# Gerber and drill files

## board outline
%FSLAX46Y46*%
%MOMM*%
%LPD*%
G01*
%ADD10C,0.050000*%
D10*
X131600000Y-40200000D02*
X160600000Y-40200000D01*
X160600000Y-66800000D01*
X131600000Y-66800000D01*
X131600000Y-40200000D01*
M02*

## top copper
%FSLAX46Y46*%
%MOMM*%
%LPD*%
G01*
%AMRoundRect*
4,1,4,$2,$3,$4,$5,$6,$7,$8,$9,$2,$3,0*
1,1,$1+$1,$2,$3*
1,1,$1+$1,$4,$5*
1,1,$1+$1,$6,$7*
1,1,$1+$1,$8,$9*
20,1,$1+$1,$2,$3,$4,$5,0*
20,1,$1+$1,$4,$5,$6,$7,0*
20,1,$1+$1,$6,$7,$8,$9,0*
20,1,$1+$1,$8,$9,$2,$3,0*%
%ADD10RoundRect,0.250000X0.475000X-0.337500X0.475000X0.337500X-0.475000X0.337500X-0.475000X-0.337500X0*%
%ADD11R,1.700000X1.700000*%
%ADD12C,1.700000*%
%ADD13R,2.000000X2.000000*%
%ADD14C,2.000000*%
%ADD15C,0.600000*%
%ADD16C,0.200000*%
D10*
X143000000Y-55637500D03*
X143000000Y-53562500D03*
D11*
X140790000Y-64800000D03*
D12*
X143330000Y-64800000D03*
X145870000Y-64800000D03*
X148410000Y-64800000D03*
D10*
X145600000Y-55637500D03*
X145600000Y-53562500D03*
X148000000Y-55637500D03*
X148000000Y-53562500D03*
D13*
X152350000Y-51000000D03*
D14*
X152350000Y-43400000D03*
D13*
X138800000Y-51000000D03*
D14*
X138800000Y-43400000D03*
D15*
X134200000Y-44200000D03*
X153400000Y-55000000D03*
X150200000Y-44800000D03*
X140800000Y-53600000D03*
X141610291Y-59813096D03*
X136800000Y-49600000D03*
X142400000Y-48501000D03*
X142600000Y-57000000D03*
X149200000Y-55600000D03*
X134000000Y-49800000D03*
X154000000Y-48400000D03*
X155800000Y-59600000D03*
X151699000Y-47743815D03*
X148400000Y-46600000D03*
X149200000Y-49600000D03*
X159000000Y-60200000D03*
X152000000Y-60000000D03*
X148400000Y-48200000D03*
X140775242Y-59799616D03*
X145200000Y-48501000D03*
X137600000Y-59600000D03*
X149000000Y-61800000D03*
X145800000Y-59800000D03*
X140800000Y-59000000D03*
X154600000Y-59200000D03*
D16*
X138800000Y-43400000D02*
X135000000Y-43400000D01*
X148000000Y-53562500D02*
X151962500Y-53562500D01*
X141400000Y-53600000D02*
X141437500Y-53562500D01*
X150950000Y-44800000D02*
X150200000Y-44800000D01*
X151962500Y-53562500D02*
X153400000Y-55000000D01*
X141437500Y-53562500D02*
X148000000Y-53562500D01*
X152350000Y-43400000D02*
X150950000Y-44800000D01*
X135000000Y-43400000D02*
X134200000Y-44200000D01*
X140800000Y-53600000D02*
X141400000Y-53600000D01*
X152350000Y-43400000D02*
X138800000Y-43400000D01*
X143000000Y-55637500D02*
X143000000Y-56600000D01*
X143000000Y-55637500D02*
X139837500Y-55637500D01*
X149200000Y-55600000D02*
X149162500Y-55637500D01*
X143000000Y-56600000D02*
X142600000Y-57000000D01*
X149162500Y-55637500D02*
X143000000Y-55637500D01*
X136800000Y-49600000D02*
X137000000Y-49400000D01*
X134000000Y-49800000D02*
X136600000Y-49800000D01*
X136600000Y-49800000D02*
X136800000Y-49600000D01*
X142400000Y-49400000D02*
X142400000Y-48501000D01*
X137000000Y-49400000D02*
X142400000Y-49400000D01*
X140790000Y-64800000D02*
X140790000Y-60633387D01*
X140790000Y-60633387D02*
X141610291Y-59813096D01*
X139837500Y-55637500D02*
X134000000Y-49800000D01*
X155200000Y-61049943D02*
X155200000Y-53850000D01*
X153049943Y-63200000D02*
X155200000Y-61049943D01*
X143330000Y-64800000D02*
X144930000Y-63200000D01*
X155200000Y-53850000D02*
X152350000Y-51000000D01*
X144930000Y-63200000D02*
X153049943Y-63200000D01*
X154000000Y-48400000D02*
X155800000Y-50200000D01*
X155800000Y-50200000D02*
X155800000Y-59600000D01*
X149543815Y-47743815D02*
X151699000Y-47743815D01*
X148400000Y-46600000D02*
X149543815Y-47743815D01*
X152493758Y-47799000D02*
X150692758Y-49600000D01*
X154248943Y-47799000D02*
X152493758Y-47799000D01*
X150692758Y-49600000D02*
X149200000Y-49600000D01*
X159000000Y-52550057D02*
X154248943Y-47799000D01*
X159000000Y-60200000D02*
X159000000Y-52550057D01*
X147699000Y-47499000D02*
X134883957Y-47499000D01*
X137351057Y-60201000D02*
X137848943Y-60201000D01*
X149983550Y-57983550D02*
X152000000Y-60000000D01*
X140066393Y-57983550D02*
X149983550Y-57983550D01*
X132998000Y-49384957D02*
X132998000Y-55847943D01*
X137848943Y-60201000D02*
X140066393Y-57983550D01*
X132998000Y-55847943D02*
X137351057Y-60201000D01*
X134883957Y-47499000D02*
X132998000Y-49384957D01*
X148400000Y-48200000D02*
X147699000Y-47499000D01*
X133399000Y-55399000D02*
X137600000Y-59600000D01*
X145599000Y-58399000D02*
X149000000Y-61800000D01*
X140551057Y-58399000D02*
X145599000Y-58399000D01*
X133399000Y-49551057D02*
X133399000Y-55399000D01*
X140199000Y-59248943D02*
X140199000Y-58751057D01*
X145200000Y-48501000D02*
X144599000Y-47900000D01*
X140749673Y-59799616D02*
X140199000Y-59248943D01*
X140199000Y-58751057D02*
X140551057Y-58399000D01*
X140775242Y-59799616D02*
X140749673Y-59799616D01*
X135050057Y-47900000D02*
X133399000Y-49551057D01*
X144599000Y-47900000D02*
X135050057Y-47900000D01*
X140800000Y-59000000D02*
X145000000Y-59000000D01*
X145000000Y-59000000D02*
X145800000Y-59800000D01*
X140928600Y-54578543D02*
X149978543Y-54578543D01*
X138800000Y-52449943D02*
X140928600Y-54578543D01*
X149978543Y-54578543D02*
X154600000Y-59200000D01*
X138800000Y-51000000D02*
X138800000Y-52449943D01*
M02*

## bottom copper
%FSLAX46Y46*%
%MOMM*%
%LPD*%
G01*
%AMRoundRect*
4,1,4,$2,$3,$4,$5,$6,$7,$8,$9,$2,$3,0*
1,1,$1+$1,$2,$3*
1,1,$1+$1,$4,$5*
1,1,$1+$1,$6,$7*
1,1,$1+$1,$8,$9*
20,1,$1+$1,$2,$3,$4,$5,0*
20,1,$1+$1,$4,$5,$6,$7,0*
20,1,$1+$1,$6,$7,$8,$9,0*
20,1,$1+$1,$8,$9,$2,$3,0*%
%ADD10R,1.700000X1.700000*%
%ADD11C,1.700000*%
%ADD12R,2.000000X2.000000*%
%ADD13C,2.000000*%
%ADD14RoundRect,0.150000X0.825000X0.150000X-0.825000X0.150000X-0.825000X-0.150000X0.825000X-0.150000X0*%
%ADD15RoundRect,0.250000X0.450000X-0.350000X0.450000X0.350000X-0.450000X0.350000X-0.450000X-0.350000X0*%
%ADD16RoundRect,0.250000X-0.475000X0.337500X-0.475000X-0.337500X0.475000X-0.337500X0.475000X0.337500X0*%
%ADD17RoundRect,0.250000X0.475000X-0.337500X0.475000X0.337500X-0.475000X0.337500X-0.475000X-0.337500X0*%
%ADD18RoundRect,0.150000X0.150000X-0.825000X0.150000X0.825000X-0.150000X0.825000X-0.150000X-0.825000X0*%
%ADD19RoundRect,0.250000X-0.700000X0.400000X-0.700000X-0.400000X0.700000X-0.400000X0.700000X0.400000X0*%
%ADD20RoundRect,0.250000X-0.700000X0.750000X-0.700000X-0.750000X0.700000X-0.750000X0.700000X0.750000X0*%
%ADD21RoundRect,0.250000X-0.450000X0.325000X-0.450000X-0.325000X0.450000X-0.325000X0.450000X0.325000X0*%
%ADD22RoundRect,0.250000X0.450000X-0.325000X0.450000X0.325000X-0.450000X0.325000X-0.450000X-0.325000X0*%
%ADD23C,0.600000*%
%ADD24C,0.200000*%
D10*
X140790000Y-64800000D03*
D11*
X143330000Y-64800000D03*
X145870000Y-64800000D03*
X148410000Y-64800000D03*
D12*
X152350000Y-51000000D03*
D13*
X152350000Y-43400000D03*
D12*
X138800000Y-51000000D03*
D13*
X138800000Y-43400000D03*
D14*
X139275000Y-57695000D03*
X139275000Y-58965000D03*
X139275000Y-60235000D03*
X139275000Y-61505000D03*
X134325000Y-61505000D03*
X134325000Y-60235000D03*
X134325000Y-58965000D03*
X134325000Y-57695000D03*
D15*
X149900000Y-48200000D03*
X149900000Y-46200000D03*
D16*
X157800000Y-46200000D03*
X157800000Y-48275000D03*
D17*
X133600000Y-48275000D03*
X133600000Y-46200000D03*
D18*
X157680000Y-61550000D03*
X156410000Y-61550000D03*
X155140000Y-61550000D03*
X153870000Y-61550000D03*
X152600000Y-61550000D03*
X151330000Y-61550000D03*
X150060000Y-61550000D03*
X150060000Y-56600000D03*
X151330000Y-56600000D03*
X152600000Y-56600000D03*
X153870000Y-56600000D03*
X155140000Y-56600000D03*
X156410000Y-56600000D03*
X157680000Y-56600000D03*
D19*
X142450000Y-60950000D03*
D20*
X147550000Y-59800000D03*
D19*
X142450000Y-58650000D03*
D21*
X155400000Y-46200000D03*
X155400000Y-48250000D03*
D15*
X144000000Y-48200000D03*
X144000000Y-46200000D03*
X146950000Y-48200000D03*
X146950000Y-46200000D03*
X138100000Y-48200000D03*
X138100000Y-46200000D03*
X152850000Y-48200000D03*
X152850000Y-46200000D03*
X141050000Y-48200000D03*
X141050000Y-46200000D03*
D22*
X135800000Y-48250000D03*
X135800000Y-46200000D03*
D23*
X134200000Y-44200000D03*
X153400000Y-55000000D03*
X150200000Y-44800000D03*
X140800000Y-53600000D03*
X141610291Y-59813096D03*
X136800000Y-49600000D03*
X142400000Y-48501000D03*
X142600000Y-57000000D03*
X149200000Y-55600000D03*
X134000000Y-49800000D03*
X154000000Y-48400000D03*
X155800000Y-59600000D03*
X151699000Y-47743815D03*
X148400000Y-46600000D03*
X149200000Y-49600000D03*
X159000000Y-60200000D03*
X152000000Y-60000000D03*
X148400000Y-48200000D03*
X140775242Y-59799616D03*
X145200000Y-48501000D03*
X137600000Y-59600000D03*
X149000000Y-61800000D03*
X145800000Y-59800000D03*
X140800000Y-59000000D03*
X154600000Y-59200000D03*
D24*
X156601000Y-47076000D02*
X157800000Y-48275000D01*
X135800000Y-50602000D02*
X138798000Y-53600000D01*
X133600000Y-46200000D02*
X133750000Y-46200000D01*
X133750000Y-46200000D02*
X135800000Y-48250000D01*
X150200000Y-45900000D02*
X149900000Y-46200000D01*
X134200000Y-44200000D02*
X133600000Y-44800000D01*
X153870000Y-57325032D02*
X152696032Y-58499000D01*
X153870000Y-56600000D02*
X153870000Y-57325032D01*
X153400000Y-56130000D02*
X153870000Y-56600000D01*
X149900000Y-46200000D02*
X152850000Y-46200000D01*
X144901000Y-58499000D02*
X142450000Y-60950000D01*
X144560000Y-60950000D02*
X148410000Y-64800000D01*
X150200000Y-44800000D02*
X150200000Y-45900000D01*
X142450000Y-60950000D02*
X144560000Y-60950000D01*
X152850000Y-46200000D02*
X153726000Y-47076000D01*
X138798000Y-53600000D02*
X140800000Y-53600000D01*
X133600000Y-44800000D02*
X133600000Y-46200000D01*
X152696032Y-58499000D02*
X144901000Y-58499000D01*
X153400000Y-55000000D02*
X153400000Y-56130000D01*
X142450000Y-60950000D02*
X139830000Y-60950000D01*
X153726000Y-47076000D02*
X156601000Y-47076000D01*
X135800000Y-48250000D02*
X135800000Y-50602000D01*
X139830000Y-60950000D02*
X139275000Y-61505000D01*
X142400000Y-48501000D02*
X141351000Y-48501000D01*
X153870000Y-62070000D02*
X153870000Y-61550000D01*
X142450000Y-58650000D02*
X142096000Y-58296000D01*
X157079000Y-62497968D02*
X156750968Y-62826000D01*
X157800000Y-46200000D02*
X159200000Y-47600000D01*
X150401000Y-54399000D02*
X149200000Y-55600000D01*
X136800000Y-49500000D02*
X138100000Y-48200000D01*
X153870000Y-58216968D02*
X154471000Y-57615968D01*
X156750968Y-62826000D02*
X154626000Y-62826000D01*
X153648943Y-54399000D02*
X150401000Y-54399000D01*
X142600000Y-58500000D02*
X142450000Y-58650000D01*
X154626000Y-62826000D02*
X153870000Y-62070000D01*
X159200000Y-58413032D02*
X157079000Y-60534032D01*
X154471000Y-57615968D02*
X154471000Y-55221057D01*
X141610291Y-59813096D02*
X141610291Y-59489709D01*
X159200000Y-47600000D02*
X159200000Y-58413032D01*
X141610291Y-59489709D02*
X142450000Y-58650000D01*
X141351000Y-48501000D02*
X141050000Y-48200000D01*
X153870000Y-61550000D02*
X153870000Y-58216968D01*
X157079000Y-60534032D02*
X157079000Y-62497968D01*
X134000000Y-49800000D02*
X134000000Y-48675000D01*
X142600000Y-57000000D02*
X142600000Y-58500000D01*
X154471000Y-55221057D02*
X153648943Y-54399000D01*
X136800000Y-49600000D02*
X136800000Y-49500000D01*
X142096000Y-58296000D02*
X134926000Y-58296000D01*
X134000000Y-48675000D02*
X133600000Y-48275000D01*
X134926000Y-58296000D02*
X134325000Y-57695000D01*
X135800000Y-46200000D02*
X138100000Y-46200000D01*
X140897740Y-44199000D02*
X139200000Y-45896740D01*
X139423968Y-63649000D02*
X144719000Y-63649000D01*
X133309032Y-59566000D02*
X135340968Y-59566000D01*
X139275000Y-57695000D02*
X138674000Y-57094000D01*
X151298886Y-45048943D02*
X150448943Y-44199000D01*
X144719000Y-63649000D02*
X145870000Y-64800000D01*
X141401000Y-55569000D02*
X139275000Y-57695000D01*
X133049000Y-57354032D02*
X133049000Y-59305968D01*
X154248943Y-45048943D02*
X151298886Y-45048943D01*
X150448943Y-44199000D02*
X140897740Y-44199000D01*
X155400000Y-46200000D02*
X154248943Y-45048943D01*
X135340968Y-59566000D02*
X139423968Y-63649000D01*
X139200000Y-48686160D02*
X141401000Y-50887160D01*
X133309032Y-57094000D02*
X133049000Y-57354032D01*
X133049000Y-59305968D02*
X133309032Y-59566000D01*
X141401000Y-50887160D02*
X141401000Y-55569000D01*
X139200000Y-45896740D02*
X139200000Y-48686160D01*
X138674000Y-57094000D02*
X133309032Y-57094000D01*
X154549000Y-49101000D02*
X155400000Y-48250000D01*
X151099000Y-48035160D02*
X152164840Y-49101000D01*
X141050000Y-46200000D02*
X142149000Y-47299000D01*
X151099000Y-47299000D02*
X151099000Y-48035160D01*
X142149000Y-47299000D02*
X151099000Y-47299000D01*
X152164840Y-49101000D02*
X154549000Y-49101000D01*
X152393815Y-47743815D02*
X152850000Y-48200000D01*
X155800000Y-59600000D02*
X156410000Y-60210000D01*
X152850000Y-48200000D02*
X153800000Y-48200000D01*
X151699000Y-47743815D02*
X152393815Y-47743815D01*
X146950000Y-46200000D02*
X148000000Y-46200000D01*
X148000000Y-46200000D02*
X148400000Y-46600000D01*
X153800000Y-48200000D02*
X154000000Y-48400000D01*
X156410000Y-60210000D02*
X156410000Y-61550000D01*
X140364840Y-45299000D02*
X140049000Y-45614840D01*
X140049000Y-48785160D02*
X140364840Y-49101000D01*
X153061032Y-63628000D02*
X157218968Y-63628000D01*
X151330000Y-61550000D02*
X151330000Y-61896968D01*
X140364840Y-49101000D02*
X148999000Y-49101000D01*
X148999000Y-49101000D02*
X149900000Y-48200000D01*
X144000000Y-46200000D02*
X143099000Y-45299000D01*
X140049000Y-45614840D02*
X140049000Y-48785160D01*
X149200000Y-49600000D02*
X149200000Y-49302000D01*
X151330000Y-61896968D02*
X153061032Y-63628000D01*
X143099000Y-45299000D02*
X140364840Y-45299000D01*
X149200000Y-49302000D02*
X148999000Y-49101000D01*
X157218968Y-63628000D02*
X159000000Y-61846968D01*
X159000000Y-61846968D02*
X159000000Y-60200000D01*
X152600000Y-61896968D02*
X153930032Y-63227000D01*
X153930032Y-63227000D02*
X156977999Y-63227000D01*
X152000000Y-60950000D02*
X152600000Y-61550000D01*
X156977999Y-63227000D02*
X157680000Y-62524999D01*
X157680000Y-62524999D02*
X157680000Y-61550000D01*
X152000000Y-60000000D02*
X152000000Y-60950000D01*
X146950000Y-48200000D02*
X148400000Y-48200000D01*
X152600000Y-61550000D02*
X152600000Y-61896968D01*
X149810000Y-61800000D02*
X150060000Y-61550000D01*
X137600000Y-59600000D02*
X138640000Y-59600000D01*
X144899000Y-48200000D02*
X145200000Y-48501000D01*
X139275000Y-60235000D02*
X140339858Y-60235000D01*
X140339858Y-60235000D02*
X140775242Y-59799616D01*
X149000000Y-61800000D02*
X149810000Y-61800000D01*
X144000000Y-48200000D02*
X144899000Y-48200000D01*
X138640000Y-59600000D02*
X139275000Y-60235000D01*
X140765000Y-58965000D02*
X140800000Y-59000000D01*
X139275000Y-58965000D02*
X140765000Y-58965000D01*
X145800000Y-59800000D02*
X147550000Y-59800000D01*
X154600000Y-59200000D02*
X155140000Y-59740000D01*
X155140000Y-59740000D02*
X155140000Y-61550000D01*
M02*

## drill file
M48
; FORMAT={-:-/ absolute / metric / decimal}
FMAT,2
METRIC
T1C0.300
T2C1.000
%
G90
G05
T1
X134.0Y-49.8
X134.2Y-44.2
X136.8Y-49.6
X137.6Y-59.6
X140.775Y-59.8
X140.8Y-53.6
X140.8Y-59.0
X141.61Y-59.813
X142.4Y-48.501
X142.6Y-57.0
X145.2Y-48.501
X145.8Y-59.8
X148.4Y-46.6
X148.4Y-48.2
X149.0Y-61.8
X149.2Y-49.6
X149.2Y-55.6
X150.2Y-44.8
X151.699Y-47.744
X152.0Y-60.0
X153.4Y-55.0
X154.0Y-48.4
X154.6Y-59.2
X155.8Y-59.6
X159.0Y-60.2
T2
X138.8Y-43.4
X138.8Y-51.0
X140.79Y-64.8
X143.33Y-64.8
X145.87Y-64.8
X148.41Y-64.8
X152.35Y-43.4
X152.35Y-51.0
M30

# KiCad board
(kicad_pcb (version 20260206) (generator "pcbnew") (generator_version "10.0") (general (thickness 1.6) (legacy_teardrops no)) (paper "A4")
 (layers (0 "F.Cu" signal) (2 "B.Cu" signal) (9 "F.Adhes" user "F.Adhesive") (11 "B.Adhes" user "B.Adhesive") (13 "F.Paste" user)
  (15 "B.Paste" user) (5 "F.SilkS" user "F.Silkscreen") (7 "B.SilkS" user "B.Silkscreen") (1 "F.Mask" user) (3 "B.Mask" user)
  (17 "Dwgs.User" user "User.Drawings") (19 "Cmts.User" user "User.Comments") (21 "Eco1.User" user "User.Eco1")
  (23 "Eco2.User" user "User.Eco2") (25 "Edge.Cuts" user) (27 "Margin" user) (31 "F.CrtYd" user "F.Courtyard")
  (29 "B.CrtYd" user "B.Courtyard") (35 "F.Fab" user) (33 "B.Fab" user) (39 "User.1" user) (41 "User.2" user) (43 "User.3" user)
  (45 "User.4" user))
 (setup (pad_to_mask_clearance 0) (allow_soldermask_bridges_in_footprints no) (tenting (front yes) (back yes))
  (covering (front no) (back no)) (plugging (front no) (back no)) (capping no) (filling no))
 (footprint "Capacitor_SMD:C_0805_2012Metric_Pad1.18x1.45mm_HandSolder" (layer "F.Cu") (at 143 54.6 90)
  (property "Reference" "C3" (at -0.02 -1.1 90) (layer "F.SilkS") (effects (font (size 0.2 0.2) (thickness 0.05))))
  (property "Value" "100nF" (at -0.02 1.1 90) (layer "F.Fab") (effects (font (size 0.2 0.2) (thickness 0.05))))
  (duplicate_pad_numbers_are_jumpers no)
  (pad "1" smd roundrect (at -1.0375 0 90) (size 1.175 1.45) (layers "F.Cu" "F.Mask" "F.Paste") (roundrect_rratio 0.212766) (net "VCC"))
  (pad "2" smd roundrect (at 1.0375 0 90) (size 1.175 1.45) (layers "F.Cu" "F.Mask" "F.Paste") (roundrect_rratio 0.212766) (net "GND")))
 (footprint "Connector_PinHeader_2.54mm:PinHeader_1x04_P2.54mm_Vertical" (layer "F.Cu") (at 140.79 64.8 90)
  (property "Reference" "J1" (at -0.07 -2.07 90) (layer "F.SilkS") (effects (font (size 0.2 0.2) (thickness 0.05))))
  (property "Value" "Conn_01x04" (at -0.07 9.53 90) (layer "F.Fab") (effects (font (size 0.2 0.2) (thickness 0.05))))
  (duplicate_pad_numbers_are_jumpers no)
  (pad "1" thru_hole rect (at 0 0 90) (size 1.7 1.7) (drill 1) (layers "*.Cu" "*.Mask") (remove_unused_layers no) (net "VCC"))
  (pad "2" thru_hole circle (at 0 2.54 90) (size 1.7 1.7) (drill 1) (layers "*.Cu" "*.Mask") (remove_unused_layers no)
   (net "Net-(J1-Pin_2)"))
  (pad "3" thru_hole circle (at 0 5.08 90) (size 1.7 1.7) (drill 1) (layers "*.Cu" "*.Mask") (remove_unused_layers no) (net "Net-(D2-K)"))
  (pad "4" thru_hole circle (at 0 7.62 90) (size 1.7 1.7) (drill 1) (layers "*.Cu" "*.Mask") (remove_unused_layers no) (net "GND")))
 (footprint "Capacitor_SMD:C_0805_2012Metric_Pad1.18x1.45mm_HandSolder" (layer "F.Cu") (at 145.6 54.6 90)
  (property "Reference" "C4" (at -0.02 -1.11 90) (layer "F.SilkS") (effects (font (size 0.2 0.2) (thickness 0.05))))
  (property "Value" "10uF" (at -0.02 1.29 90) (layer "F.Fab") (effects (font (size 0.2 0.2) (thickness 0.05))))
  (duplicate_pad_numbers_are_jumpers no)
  (pad "1" smd roundrect (at -1.0375 0 90) (size 1.175 1.45) (layers "F.Cu" "F.Mask" "F.Paste") (roundrect_rratio 0.212766) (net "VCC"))
  (pad "2" smd roundrect (at 1.0375 0 90) (size 1.175 1.45) (layers "F.Cu" "F.Mask" "F.Paste") (roundrect_rratio 0.212766) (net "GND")))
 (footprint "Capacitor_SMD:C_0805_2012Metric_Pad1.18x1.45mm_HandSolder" (layer "F.Cu") (at 148 54.6 90)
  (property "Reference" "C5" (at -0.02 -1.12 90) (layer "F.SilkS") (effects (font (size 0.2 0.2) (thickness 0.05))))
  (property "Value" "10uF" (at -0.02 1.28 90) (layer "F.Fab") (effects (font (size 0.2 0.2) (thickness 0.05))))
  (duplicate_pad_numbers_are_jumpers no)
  (pad "1" smd roundrect (at -1.0375 0 90) (size 1.175 1.45) (layers "F.Cu" "F.Mask" "F.Paste") (roundrect_rratio 0.212766) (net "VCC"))
  (pad "2" smd roundrect (at 1.0375 0 90) (size 1.175 1.45) (layers "F.Cu" "F.Mask" "F.Paste") (roundrect_rratio 0.212766) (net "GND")))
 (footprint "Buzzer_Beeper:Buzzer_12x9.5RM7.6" (layer "F.Cu") (at 152.35 51 90)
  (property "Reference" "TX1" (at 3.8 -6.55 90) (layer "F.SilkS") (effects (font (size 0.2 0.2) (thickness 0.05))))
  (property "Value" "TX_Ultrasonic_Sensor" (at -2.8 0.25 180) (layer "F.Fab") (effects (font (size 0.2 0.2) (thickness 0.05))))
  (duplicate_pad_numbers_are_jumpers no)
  (pad "1" thru_hole rect (at 0 0 90) (size 2 2) (drill 1) (layers "*.Cu" "*.Mask") (remove_unused_layers no) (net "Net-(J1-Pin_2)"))
  (pad "2" thru_hole circle (at 7.6 0 90) (size 2 2) (drill 1) (layers "*.Cu" "*.Mask") (remove_unused_layers no) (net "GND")))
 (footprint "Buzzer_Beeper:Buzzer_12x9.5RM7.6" (layer "F.Cu") (at 138.8 51 90)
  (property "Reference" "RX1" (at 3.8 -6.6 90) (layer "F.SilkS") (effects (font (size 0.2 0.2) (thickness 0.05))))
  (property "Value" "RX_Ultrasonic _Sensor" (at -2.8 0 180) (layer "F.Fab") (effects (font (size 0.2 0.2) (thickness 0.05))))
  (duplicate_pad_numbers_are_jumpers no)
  (pad "1" thru_hole rect (at 0 0 90) (size 2 2) (drill 1) (layers "*.Cu" "*.Mask") (remove_unused_layers no) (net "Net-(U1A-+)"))
  (pad "2" thru_hole circle (at 7.6 0 90) (size 2 2) (drill 1) (layers "*.Cu" "*.Mask") (remove_unused_layers no) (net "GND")))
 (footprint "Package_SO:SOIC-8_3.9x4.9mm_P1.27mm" (layer "B.Cu") (at 136.8 59.6 180)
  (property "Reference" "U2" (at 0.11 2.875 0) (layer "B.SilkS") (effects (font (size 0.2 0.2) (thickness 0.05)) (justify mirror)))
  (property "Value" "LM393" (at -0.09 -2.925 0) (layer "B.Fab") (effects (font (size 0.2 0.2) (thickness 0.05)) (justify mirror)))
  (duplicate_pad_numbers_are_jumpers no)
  (pad "1" smd roundrect (at -2.475 1.905 180) (size 1.95 0.6) (layers "B.Cu" "B.Mask" "B.Paste") (roundrect_rratio 0.25) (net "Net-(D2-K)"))
  (pad "2" smd roundrect (at -2.475 0.635 180) (size 1.95 0.6) (layers "B.Cu" "B.Mask" "B.Paste") (roundrect_rratio 0.25)
   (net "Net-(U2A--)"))
  (pad "3" smd roundrect (at -2.475 -0.635 180) (size 1.95 0.6) (layers "B.Cu" "B.Mask" "B.Paste") (roundrect_rratio 0.25)
   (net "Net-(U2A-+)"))
  (pad "4" smd roundrect (at -2.475 -1.905 180) (size 1.95 0.6) (layers "B.Cu" "B.Mask" "B.Paste") (roundrect_rratio 0.25) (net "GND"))
  (pad "5" smd roundrect (at 2.475 -1.905 180) (size 1.95 0.6) (layers "B.Cu" "B.Mask" "B.Paste") (roundrect_rratio 0.25))
  (pad "6" smd roundrect (at 2.475 -0.635 180) (size 1.95 0.6) (layers "B.Cu" "B.Mask" "B.Paste") (roundrect_rratio 0.25))
  (pad "7" smd roundrect (at 2.475 0.635 180) (size 1.95 0.6) (layers "B.Cu" "B.Mask" "B.Paste") (roundrect_rratio 0.25))
  (pad "8" smd roundrect (at 2.475 1.905 180) (size 1.95 0.6) (layers "B.Cu" "B.Mask" "B.Paste") (roundrect_rratio 0.25) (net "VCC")))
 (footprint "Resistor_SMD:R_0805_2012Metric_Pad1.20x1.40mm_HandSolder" (layer "B.Cu") (at 149.9 47.2 90)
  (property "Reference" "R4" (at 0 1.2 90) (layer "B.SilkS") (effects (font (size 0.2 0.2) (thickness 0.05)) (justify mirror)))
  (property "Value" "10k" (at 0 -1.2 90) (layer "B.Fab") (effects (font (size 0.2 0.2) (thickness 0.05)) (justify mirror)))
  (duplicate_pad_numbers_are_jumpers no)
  (pad "1" smd roundrect (at -1 0 90) (size 1.2 1.4) (layers "B.Cu" "B.Mask" "B.Paste") (roundrect_rratio 0.208333) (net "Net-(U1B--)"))
  (pad "2" smd roundrect (at 1 0 90) (size 1.2 1.4) (layers "B.Cu" "B.Mask" "B.Paste") (roundrect_rratio 0.208333) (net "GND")))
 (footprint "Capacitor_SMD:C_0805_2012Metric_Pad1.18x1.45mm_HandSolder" (layer "B.Cu") (at 157.8 47.2375 -90)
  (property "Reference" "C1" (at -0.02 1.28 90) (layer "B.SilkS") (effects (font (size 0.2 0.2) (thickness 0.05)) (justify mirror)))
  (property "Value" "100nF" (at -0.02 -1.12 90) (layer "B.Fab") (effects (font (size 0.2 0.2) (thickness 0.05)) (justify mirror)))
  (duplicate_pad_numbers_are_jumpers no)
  (pad "1" smd roundrect (at -1.0375 0 270) (size 1.175 1.45) (layers "B.Cu" "B.Mask" "B.Paste") (roundrect_rratio 0.212766) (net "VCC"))
  (pad "2" smd roundrect (at 1.0375 0 270) (size 1.175 1.45) (layers "B.Cu" "B.Mask" "B.Paste") (roundrect_rratio 0.212766) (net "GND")))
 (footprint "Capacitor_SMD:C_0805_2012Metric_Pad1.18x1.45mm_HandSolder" (layer "B.Cu") (at 133.6 47.2375 90)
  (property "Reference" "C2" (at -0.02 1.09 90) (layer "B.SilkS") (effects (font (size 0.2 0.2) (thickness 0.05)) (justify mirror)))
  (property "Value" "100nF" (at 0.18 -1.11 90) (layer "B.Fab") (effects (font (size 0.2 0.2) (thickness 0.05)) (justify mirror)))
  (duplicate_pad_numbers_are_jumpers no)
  (pad "1" smd roundrect (at -1.0375 0 90) (size 1.175 1.45) (layers "B.Cu" "B.Mask" "B.Paste") (roundrect_rratio 0.212766) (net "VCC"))
  (pad "2" smd roundrect (at 1.0375 0 90) (size 1.175 1.45) (layers "B.Cu" "B.Mask" "B.Paste") (roundrect_rratio 0.212766) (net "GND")))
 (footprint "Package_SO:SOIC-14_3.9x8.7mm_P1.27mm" (layer "B.Cu") (at 153.87 59.075 90)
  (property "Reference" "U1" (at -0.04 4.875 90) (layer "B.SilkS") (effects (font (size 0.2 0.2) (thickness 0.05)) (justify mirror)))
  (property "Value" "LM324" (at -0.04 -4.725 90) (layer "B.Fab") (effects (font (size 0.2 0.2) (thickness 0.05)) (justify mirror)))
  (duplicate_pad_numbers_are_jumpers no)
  (pad "1" smd roundrect (at -2.475 3.81 90) (size 1.95 0.6) (layers "B.Cu" "B.Mask" "B.Paste") (roundrect_rratio 0.25) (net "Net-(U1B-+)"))
  (pad "2" smd roundrect (at -2.475 2.54 90) (size 1.95 0.6) (layers "B.Cu" "B.Mask" "B.Paste") (roundrect_rratio 0.25) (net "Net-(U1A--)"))
  (pad "3" smd roundrect (at -2.475 1.27 90) (size 1.95 0.6) (layers "B.Cu" "B.Mask" "B.Paste") (roundrect_rratio 0.25) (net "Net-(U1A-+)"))
  (pad "4" smd roundrect (at -2.475 0 90) (size 1.95 0.6) (layers "B.Cu" "B.Mask" "B.Paste") (roundrect_rratio 0.25) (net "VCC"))
  (pad "5" smd roundrect (at -2.475 -1.27 90) (size 1.95 0.6) (layers "B.Cu" "B.Mask" "B.Paste") (roundrect_rratio 0.25) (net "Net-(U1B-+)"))
  (pad "6" smd roundrect (at -2.475 -2.54 90) (size 1.95 0.6) (layers "B.Cu" "B.Mask" "B.Paste") (roundrect_rratio 0.25) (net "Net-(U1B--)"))
  (pad "7" smd roundrect (at -2.475 -3.81 90) (size 1.95 0.6) (layers "B.Cu" "B.Mask" "B.Paste") (roundrect_rratio 0.25) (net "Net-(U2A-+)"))
  (pad "8" smd roundrect (at 2.475 -3.81 90) (size 1.95 0.6) (layers "B.Cu" "B.Mask" "B.Paste") (roundrect_rratio 0.25))
  (pad "9" smd roundrect (at 2.475 -2.54 90) (size 1.95 0.6) (layers "B.Cu" "B.Mask" "B.Paste") (roundrect_rratio 0.25))
  (pad "10" smd roundrect (at 2.475 -1.27 90) (size 1.95 0.6) (layers "B.Cu" "B.Mask" "B.Paste") (roundrect_rratio 0.25))
  (pad "11" smd roundrect (at 2.475 0 90) (size 1.95 0.6) (layers "B.Cu" "B.Mask" "B.Paste") (roundrect_rratio 0.25) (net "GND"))
  (pad "12" smd roundrect (at 2.475 1.27 90) (size 1.95 0.6) (layers "B.Cu" "B.Mask" "B.Paste") (roundrect_rratio 0.25))
  (pad "13" smd roundrect (at 2.475 2.54 90) (size 1.95 0.6) (layers "B.Cu" "B.Mask" "B.Paste") (roundrect_rratio 0.25))
  (pad "14" smd roundrect (at 2.475 3.81 90) (size 1.95 0.6) (layers "B.Cu" "B.Mask" "B.Paste") (roundrect_rratio 0.25)))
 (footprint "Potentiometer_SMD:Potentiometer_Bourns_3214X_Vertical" (layer "B.Cu") (at 145 59.8 -90)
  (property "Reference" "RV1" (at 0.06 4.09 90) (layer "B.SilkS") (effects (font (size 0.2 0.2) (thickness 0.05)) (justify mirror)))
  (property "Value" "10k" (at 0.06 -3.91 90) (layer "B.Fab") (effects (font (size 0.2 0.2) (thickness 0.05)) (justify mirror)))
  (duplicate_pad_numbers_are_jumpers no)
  (pad "1" smd roundrect (at 1.15 2.55 270) (size 1.3 1.9) (layers "B.Cu" "B.Mask" "B.Paste") (roundrect_rratio 0.192308) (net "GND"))
  (pad "2" smd roundrect (at 0 -2.55 270) (size 2 1.9) (layers "B.Cu" "B.Mask" "B.Paste") (roundrect_rratio 0.131579) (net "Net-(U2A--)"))
  (pad "3" smd roundrect (at -1.15 2.55 270) (size 1.3 1.9) (layers "B.Cu" "B.Mask" "B.Paste") (roundrect_rratio 0.192308) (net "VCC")))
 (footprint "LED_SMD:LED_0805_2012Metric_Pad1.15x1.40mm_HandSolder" (layer "B.Cu") (at 155.4 47.225 -90)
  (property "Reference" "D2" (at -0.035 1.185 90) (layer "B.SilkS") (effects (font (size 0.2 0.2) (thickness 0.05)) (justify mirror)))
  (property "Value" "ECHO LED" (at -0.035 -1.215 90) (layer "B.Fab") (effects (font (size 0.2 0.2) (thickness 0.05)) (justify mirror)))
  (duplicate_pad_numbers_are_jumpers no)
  (pad "1" smd roundrect (at -1.025 0 270) (size 1.15 1.4) (layers "B.Cu" "B.Mask" "B.Paste") (roundrect_rratio 0.217391) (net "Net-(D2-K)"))
  (pad "2" smd roundrect (at 1.025 0 270) (size 1.15 1.4) (layers "B.Cu" "B.Mask" "B.Paste") (roundrect_rratio 0.217391) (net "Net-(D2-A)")))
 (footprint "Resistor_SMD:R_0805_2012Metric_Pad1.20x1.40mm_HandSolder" (layer "B.Cu") (at 144 47.2 90)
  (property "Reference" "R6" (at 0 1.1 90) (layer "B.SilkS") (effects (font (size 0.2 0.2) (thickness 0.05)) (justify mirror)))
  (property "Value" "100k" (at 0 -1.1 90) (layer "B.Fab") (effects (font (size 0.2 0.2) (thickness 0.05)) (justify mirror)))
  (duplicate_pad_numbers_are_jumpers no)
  (pad "1" smd roundrect (at -1 0 90) (size 1.2 1.4) (layers "B.Cu" "B.Mask" "B.Paste") (roundrect_rratio 0.208333) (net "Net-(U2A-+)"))
  (pad "2" smd roundrect (at 1 0 90) (size 1.2 1.4) (layers "B.Cu" "B.Mask" "B.Paste") (roundrect_rratio 0.208333) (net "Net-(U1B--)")))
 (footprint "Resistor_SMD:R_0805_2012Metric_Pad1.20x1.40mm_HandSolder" (layer "B.Cu") (at 146.95 47.2 90)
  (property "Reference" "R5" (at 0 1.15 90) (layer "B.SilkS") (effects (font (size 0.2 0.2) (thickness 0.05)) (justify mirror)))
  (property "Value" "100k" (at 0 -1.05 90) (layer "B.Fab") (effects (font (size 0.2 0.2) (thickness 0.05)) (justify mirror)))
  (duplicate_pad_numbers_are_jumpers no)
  (pad "1" smd roundrect (at -1 0 90) (size 1.2 1.4) (layers "B.Cu" "B.Mask" "B.Paste") (roundrect_rratio 0.208333) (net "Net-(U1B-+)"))
  (pad "2" smd roundrect (at 1 0 90) (size 1.2 1.4) (layers "B.Cu" "B.Mask" "B.Paste") (roundrect_rratio 0.208333) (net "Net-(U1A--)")))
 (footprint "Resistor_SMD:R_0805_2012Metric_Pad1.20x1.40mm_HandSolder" (layer "B.Cu") (at 138.1 47.2 90)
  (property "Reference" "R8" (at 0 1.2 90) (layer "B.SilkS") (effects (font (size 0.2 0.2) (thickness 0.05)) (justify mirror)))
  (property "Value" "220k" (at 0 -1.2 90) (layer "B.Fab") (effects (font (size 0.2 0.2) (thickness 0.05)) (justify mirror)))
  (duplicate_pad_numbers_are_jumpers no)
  (pad "1" smd roundrect (at -1 0 90) (size 1.2 1.4) (layers "B.Cu" "B.Mask" "B.Paste") (roundrect_rratio 0.208333) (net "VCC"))
  (pad "2" smd roundrect (at 1 0 90) (size 1.2 1.4) (layers "B.Cu" "B.Mask" "B.Paste") (roundrect_rratio 0.208333) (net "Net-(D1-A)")))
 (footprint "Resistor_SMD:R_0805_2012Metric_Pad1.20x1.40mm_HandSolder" (layer "B.Cu") (at 152.85 47.2 90)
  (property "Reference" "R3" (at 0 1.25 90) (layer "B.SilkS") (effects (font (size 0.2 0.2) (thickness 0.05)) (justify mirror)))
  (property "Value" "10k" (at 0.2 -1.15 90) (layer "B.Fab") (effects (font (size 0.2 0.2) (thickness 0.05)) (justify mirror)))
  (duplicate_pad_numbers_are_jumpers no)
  (pad "1" smd roundrect (at -1 0 90) (size 1.2 1.4) (layers "B.Cu" "B.Mask" "B.Paste") (roundrect_rratio 0.208333) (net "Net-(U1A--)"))
  (pad "2" smd roundrect (at 1 0 90) (size 1.2 1.4) (layers "B.Cu" "B.Mask" "B.Paste") (roundrect_rratio 0.208333) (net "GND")))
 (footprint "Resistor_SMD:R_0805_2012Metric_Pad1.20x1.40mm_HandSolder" (layer "B.Cu") (at 141.05 47.2 90)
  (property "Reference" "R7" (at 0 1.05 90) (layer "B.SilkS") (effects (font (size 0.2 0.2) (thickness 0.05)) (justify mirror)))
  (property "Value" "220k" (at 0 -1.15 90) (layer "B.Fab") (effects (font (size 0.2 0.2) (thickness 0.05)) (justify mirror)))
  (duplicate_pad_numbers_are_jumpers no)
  (pad "1" smd roundrect (at -1 0 90) (size 1.2 1.4) (layers "B.Cu" "B.Mask" "B.Paste") (roundrect_rratio 0.208333) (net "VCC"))
  (pad "2" smd roundrect (at 1 0 90) (size 1.2 1.4) (layers "B.Cu" "B.Mask" "B.Paste") (roundrect_rratio 0.208333) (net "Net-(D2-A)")))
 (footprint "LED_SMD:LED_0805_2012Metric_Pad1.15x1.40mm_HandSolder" (layer "B.Cu") (at 135.8 47.225 90)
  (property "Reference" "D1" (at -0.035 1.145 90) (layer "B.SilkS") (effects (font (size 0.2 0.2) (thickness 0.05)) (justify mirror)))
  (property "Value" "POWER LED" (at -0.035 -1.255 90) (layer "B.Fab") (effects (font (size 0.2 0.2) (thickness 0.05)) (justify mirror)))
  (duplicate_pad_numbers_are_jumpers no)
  (pad "1" smd roundrect (at -1.025 0 90) (size 1.15 1.4) (layers "B.Cu" "B.Mask" "B.Paste") (roundrect_rratio 0.217391) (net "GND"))
  (pad "2" smd roundrect (at 1.025 0 90) (size 1.15 1.4) (layers "B.Cu" "B.Mask" "B.Paste") (roundrect_rratio 0.217391) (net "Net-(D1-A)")))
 (gr_rect (start 131.6 40.2) (end 160.6 66.8) (stroke (width 0.05) (type default)) (fill no) (layer "Edge.Cuts"))
 (segment (start 138.8 43.4) (end 135 43.4) (width 0.2) (layer "F.Cu") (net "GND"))
 (segment (start 148 53.5625) (end 151.9625 53.5625) (width 0.2) (layer "F.Cu") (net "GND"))
 (segment (start 141.4 53.6) (end 141.4375 53.5625) (width 0.2) (layer "F.Cu") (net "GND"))
 (segment (start 150.95 44.8) (end 150.2 44.8) (width 0.2) (layer "F.Cu") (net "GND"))
 (segment (start 151.9625 53.5625) (end 153.4 55) (width 0.2) (layer "F.Cu") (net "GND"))
 (segment (start 141.4375 53.5625) (end 148 53.5625) (width 0.2) (layer "F.Cu") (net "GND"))
 (segment (start 152.35 43.4) (end 150.95 44.8) (width 0.2) (layer "F.Cu") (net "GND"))
 (segment (start 135 43.4) (end 134.2 44.2) (width 0.2) (layer "F.Cu") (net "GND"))
 (segment (start 140.8 53.6) (end 141.4 53.6) (width 0.2) (layer "F.Cu") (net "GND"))
 (segment (start 152.35 43.4) (end 138.8 43.4) (width 0.2) (layer "F.Cu") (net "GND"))
 (via (at 134.2 44.2) (size 0.6) (drill 0.3) (layers "F.Cu" "B.Cu") (capping no) (covering (front no) (back no))
  (plugging (front no) (back no)) (filling no) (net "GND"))
 (via (at 153.4 55) (size 0.6) (drill 0.3) (layers "F.Cu" "B.Cu") (capping no) (covering (front no) (back no))
  (plugging (front no) (back no)) (filling no) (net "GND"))
 (via (at 150.2 44.8) (size 0.6) (drill 0.3) (layers "F.Cu" "B.Cu") (capping no) (covering (front no) (back no))
  (plugging (front no) (back no)) (filling no) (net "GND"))
 (via (at 140.8 53.6) (size 0.6) (drill 0.3) (layers "F.Cu" "B.Cu") (capping no) (covering (front no) (back no))
  (plugging (front no) (back no)) (filling no) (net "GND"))
 (segment (start 156.601 47.076) (end 157.8 48.275) (width 0.2) (layer "B.Cu") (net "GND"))
 (segment (start 135.8 50.602) (end 138.798 53.6) (width 0.2) (layer "B.Cu") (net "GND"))
 (segment (start 133.6 46.2) (end 133.75 46.2) (width 0.2) (layer "B.Cu") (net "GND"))
 (segment (start 133.75 46.2) (end 135.8 48.25) (width 0.2) (layer "B.Cu") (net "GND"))
 (segment (start 150.2 45.9) (end 149.9 46.2) (width 0.2) (layer "B.Cu") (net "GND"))
 (segment (start 134.2 44.2) (end 133.6 44.8) (width 0.2) (layer "B.Cu") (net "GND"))
 (segment (start 153.87 57.325032) (end 152.696032 58.499) (width 0.2) (layer "B.Cu") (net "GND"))
 (segment (start 153.87 56.6) (end 153.87 57.325032) (width 0.2) (layer "B.Cu") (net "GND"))
 (segment (start 153.4 56.13) (end 153.87 56.6) (width 0.2) (layer "B.Cu") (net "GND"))
 (segment (start 149.9 46.2) (end 152.85 46.2) (width 0.2) (layer "B.Cu") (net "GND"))
 (segment (start 144.901 58.499) (end 142.45 60.95) (width 0.2) (layer "B.Cu") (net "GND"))
 (segment (start 144.56 60.95) (end 148.41 64.8) (width 0.2) (layer "B.Cu") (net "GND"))
 (segment (start 150.2 44.8) (end 150.2 45.9) (width 0.2) (layer "B.Cu") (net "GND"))
 (segment (start 142.45 60.95) (end 144.56 60.95) (width 0.2) (layer "B.Cu") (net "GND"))
 (segment (start 152.85 46.2) (end 153.726 47.076) (width 0.2) (layer "B.Cu") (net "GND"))
 (segment (start 138.798 53.6) (end 140.8 53.6) (width 0.2) (layer "B.Cu") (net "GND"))
 (segment (start 133.6 44.8) (end 133.6 46.2) (width 0.2) (layer "B.Cu") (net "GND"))
 (segment (start 152.696032 58.499) (end 144.901 58.499) (width 0.2) (layer "B.Cu") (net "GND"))
 (segment (start 153.4 55) (end 153.4 56.13) (width 0.2) (layer "B.Cu") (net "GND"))
 (segment (start 142.45 60.95) (end 139.83 60.95) (width 0.2) (layer "B.Cu") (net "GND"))
 (segment (start 153.726 47.076) (end 156.601 47.076) (width 0.2) (layer "B.Cu") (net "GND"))
 (segment (start 135.8 48.25) (end 135.8 50.602) (width 0.2) (layer "B.Cu") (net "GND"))
 (segment (start 139.83 60.95) (end 139.275 61.505) (width 0.2) (layer "B.Cu") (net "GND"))
 (segment (start 143 55.6375) (end 143 56.6) (width 0.2) (layer "F.Cu") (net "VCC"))
 (segment (start 143 55.6375) (end 139.8375 55.6375) (width 0.2) (layer "F.Cu") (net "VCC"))
 (segment (start 149.2 55.6) (end 149.1625 55.6375) (width 0.2) (layer "F.Cu") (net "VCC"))
 (segment (start 143 56.6) (end 142.6 57) (width 0.2) (layer "F.Cu") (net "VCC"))
 (segment (start 149.1625 55.6375) (end 143 55.6375) (width 0.2) (layer "F.Cu") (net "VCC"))
 (segment (start 136.8 49.6) (end 137 49.4) (width 0.2) (layer "F.Cu") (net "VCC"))
 (segment (start 134 49.8) (end 136.6 49.8) (width 0.2) (layer "F.Cu") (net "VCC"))
 (segment (start 136.6 49.8) (end 136.8 49.6) (width 0.2) (layer "F.Cu") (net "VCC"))
 (segment (start 142.4 49.4) (end 142.4 48.501) (width 0.2) (layer "F.Cu") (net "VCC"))
 (segment (start 137 49.4) (end 142.4 49.4) (width 0.2) (layer "F.Cu") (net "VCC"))
 (segment (start 140.79 64.8) (end 140.79 60.633387) (width 0.2) (layer "F.Cu") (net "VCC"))
 (segment (start 140.79 60.633387) (end 141.610291 59.813096) (width 0.2) (layer "F.Cu") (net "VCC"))
 (segment (start 139.8375 55.6375) (end 134 49.8) (width 0.2) (layer "F.Cu") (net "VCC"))
 (via (at 141.610291 59.813096) (size 0.6) (drill 0.3) (layers "F.Cu" "B.Cu") (capping no) (covering (front no) (back no))
  (plugging (front no) (back no)) (filling no) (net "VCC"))
 (via (at 136.8 49.6) (size 0.6) (drill 0.3) (layers "F.Cu" "B.Cu") (capping no) (covering (front no) (back no))
  (plugging (front no) (back no)) (filling no) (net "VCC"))
 (via (at 142.4 48.501) (size 0.6) (drill 0.3) (layers "F.Cu" "B.Cu") (capping no) (covering (front no) (back no))
  (plugging (front no) (back no)) (filling no) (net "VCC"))
 (via (at 142.6 57) (size 0.6) (drill 0.3) (layers "F.Cu" "B.Cu") (capping no) (covering (front no) (back no))
  (plugging (front no) (back no)) (filling no) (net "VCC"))
 (via (at 149.2 55.6) (size 0.6) (drill 0.3) (layers "F.Cu" "B.Cu") (capping no) (covering (front no) (back no))
  (plugging (front no) (back no)) (filling no) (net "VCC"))
 (via (at 134 49.8) (size 0.6) (drill 0.3) (layers "F.Cu" "B.Cu") (capping no) (covering (front no) (back no))
  (plugging (front no) (back no)) (filling no) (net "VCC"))
 (segment (start 142.4 48.501) (end 141.351 48.501) (width 0.2) (layer "B.Cu") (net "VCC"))
 (segment (start 153.87 62.07) (end 153.87 61.55) (width 0.2) (layer "B.Cu") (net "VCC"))
 (segment (start 142.45 58.65) (end 142.096 58.296) (width 0.2) (layer "B.Cu") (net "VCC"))
 (segment (start 157.079 62.497968) (end 156.750968 62.826) (width 0.2) (layer "B.Cu") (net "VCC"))
 (segment (start 157.8 46.2) (end 159.2 47.6) (width 0.2) (layer "B.Cu") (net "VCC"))
 (segment (start 150.401 54.399) (end 149.2 55.6) (width 0.2) (layer "B.Cu") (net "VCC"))
 (segment (start 136.8 49.5) (end 138.1 48.2) (width 0.2) (layer "B.Cu") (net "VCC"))
 (segment (start 153.87 58.216968) (end 154.471 57.615968) (width 0.2) (layer "B.Cu") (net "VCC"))
 (segment (start 156.750968 62.826) (end 154.626 62.826) (width 0.2) (layer "B.Cu") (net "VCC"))
 (segment (start 153.648943 54.399) (end 150.401 54.399) (width 0.2) (layer "B.Cu") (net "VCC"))
 (segment (start 142.6 58.5) (end 142.45 58.65) (width 0.2) (layer "B.Cu") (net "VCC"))
 (segment (start 154.626 62.826) (end 153.87 62.07) (width 0.2) (layer "B.Cu") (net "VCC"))
 (segment (start 159.2 58.413032) (end 157.079 60.534032) (width 0.2) (layer "B.Cu") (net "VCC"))
 (segment (start 154.471 57.615968) (end 154.471 55.221057) (width 0.2) (layer "B.Cu") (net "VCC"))
 (segment (start 141.610291 59.813096) (end 141.610291 59.489709) (width 0.2) (layer "B.Cu") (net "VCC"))
 (segment (start 159.2 47.6) (end 159.2 58.413032) (width 0.2) (layer "B.Cu") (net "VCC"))
 (segment (start 141.610291 59.489709) (end 142.45 58.65) (width 0.2) (layer "B.Cu") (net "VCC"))
 (segment (start 141.351 48.501) (end 141.05 48.2) (width 0.2) (layer "B.Cu") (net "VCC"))
 (segment (start 153.87 61.55) (end 153.87 58.216968) (width 0.2) (layer "B.Cu") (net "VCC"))
 (segment (start 157.079 60.534032) (end 157.079 62.497968) (width 0.2) (layer "B.Cu") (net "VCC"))
 (segment (start 134 49.8) (end 134 48.675) (width 0.2) (layer "B.Cu") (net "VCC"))
 (segment (start 142.6 57) (end 142.6 58.5) (width 0.2) (layer "B.Cu") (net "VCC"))
 (segment (start 154.471 55.221057) (end 153.648943 54.399) (width 0.2) (layer "B.Cu") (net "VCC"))
 (segment (start 136.8 49.6) (end 136.8 49.5) (width 0.2) (layer "B.Cu") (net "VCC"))
 (segment (start 142.096 58.296) (end 134.926 58.296) (width 0.2) (layer "B.Cu") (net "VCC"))
 (segment (start 134 48.675) (end 133.6 48.275) (width 0.2) (layer "B.Cu") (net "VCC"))
 (segment (start 134.926 58.296) (end 134.325 57.695) (width 0.2) (layer "B.Cu") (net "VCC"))
 (segment (start 135.8 46.2) (end 138.1 46.2) (width 0.2) (layer "B.Cu") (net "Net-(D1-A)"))
 (segment (start 140.89774 44.199) (end 139.2 45.89674) (width 0.2) (layer "B.Cu") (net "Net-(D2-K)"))
 (segment (start 139.423968 63.649) (end 144.719 63.649) (width 0.2) (layer "B.Cu") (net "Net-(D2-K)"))
 (segment (start 133.309032 59.566) (end 135.340968 59.566) (width 0.2) (layer "B.Cu") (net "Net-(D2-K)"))
 (segment (start 139.275 57.695) (end 138.674 57.094) (width 0.2) (layer "B.Cu") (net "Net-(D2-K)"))
 (segment (start 151.298886 45.048943) (end 150.448943 44.199) (width 0.2) (layer "B.Cu") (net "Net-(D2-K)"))
 (segment (start 144.719 63.649) (end 145.87 64.8) (width 0.2) (layer "B.Cu") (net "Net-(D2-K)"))
 (segment (start 141.401 55.569) (end 139.275 57.695) (width 0.2) (layer "B.Cu") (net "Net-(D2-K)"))
 (segment (start 133.049 57.354032) (end 133.049 59.305968) (width 0.2) (layer "B.Cu") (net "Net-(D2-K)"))
 (segment (start 154.248943 45.048943) (end 151.298886 45.048943) (width 0.2) (layer "B.Cu") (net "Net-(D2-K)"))
 (segment (start 150.448943 44.199) (end 140.89774 44.199) (width 0.2) (layer "B.Cu") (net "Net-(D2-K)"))
 (segment (start 155.4 46.2) (end 154.248943 45.048943) (width 0.2) (layer "B.Cu") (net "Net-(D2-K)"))
 (segment (start 135.340968 59.566) (end 139.423968 63.649) (width 0.2) (layer "B.Cu") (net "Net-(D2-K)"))
 (segment (start 139.2 48.68616) (end 141.401 50.88716) (width 0.2) (layer "B.Cu") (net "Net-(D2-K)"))
 (segment (start 133.309032 57.094) (end 133.049 57.354032) (width 0.2) (layer "B.Cu") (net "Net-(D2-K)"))
 (segment (start 133.049 59.305968) (end 133.309032 59.566) (width 0.2) (layer "B.Cu") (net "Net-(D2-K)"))
 (segment (start 141.401 50.88716) (end 141.401 55.569) (width 0.2) (layer "B.Cu") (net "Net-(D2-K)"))
 (segment (start 139.2 45.89674) (end 139.2 48.68616) (width 0.2) (layer "B.Cu") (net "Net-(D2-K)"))
 (segment (start 138.674 57.094) (end 133.309032 57.094) (width 0.2) (layer "B.Cu") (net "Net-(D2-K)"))
 (segment (start 154.549 49.101) (end 155.4 48.25) (width 0.2) (layer "B.Cu") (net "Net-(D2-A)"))
 (segment (start 151.099 48.03516) (end 152.16484 49.101) (width 0.2) (layer "B.Cu") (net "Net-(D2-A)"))
 (segment (start 141.05 46.2) (end 142.149 47.299) (width 0.2) (layer "B.Cu") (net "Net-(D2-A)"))
 (segment (start 151.099 47.299) (end 151.099 48.03516) (width 0.2) (layer "B.Cu") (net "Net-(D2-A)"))
 (segment (start 142.149 47.299) (end 151.099 47.299) (width 0.2) (layer "B.Cu") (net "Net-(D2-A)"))
 (segment (start 152.16484 49.101) (end 154.549 49.101) (width 0.2) (layer "B.Cu") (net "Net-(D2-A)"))
 (segment (start 155.2 61.049943) (end 155.2 53.85) (width 0.2) (layer "F.Cu") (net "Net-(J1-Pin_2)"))
 (segment (start 153.049943 63.2) (end 155.2 61.049943) (width 0.2) (layer "F.Cu") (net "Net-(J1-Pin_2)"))
 (segment (start 143.33 64.8) (end 144.93 63.2) (width 0.2) (layer "F.Cu") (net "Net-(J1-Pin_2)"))
 (segment (start 155.2 53.85) (end 152.35 51) (width 0.2) (layer "F.Cu") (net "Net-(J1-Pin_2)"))
 (segment (start 144.93 63.2) (end 153.049943 63.2) (width 0.2) (layer "F.Cu") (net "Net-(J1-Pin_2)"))
 (segment (start 154 48.4) (end 155.8 50.2) (width 0.2) (layer "F.Cu") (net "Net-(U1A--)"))
 (segment (start 155.8 50.2) (end 155.8 59.6) (width 0.2) (layer "F.Cu") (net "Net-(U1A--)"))
 (segment (start 149.543815 47.743815) (end 151.699 47.743815) (width 0.2) (layer "F.Cu") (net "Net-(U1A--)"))
 (segment (start 148.4 46.6) (end 149.543815 47.743815) (width 0.2) (layer "F.Cu") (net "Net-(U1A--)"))
 (via (at 154 48.4) (size 0.6) (drill 0.3) (layers "F.Cu" "B.Cu") (capping no) (covering (front no) (back no))
  (plugging (front no) (back no)) (filling no) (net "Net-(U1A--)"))
 (via (at 155.8 59.6) (size 0.6) (drill 0.3) (layers "F.Cu" "B.Cu") (capping no) (covering (front no) (back no))
  (plugging (front no) (back no)) (filling no) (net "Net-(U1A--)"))
 (via (at 151.699 47.743815) (size 0.6) (drill 0.3) (layers "F.Cu" "B.Cu") (capping no) (covering (front no) (back no))
  (plugging (front no) (back no)) (filling no) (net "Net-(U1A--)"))
 (via (at 148.4 46.6) (size 0.6) (drill 0.3) (layers "F.Cu" "B.Cu") (capping no) (covering (front no) (back no))
  (plugging (front no) (back no)) (filling no) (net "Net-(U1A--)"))
 (segment (start 152.393815 47.743815) (end 152.85 48.2) (width 0.2) (layer "B.Cu") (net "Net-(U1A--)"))
 (segment (start 155.8 59.6) (end 156.41 60.21) (width 0.2) (layer "B.Cu") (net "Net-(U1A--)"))
 (segment (start 152.85 48.2) (end 153.8 48.2) (width 0.2) (layer "B.Cu") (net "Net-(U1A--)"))
 (segment (start 151.699 47.743815) (end 152.393815 47.743815) (width 0.2) (layer "B.Cu") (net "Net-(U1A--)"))
 (segment (start 146.95 46.2) (end 148 46.2) (width 0.2) (layer "B.Cu") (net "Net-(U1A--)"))
 (segment (start 148 46.2) (end 148.4 46.6) (width 0.2) (layer "B.Cu") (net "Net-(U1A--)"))
 (segment (start 153.8 48.2) (end 154 48.4) (width 0.2) (layer "B.Cu") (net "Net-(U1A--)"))
 (segment (start 156.41 60.21) (end 156.41 61.55) (width 0.2) (layer "B.Cu") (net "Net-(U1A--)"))
 (segment (start 152.493758 47.799) (end 150.692758 49.6) (width 0.2) (layer "F.Cu") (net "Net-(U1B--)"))
 (segment (start 154.248943 47.799) (end 152.493758 47.799) (width 0.2) (layer "F.Cu") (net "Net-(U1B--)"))
 (segment (start 150.692758 49.6) (end 149.2 49.6) (width 0.2) (layer "F.Cu") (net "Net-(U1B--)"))
 (segment (start 159 52.550057) (end 154.248943 47.799) (width 0.2) (layer "F.Cu") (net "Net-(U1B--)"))
 (segment (start 159 60.2) (end 159 52.550057) (width 0.2) (layer "F.Cu") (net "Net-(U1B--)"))
 (via (at 149.2 49.6) (size 0.6) (drill 0.3) (layers "F.Cu" "B.Cu") (capping no) (covering (front no) (back no))
  (plugging (front no) (back no)) (filling no) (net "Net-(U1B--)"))
 (via (at 159 60.2) (size 0.6) (drill 0.3) (layers "F.Cu" "B.Cu") (capping no) (covering (front no) (back no))
  (plugging (front no) (back no)) (filling no) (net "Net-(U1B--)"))
 (segment (start 140.36484 45.299) (end 140.049 45.61484) (width 0.2) (layer "B.Cu") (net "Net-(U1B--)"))
 (segment (start 140.049 48.78516) (end 140.36484 49.101) (width 0.2) (layer "B.Cu") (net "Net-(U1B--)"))
 (segment (start 153.061032 63.628) (end 157.218968 63.628) (width 0.2) (layer "B.Cu") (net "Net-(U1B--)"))
 (segment (start 151.33 61.55) (end 151.33 61.896968) (width 0.2) (layer "B.Cu") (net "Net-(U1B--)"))
 (segment (start 140.36484 49.101) (end 148.999 49.101) (width 0.2) (layer "B.Cu") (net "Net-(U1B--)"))
 (segment (start 148.999 49.101) (end 149.9 48.2) (width 0.2) (layer "B.Cu") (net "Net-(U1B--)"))
 (segment (start 144 46.2) (end 143.099 45.299) (width 0.2) (layer "B.Cu") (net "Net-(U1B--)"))
 (segment (start 140.049 45.61484) (end 140.049 48.78516) (width 0.2) (layer "B.Cu") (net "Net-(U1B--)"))
 (segment (start 149.2 49.6) (end 149.2 49.302) (width 0.2) (layer "B.Cu") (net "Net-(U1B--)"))
 (segment (start 151.33 61.896968) (end 153.061032 63.628) (width 0.2) (layer "B.Cu") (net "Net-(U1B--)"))
 (segment (start 143.099 45.299) (end 140.36484 45.299) (width 0.2) (layer "B.Cu") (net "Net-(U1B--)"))
 (segment (start 149.2 49.302) (end 148.999 49.101) (width 0.2) (layer "B.Cu") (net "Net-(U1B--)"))
 (segment (start 157.218968 63.628) (end 159 61.846968) (width 0.2) (layer "B.Cu") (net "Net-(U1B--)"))
 (segment (start 159 61.846968) (end 159 60.2) (width 0.2) (layer "B.Cu") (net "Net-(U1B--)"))
 (segment (start 147.699 47.499) (end 134.883957 47.499) (width 0.2) (layer "F.Cu") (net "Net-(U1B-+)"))
 (segment (start 137.351057 60.201) (end 137.848943 60.201) (width 0.2) (layer "F.Cu") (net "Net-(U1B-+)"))
 (segment (start 149.98355 57.98355) (end 152 60) (width 0.2) (layer "F.Cu") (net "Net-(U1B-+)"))
 (segment (start 140.066393 57.98355) (end 149.98355 57.98355) (width 0.2) (layer "F.Cu") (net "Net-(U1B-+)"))
 (segment (start 132.998 49.384957) (end 132.998 55.847943) (width 0.2) (layer "F.Cu") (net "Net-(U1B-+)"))
 (segment (start 137.848943 60.201) (end 140.066393 57.98355) (width 0.2) (layer "F.Cu") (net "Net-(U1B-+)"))
 (segment (start 132.998 55.847943) (end 137.351057 60.201) (width 0.2) (layer "F.Cu") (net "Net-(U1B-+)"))
 (segment (start 134.883957 47.499) (end 132.998 49.384957) (width 0.2) (layer "F.Cu") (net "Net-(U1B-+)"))
 (segment (start 148.4 48.2) (end 147.699 47.499) (width 0.2) (layer "F.Cu") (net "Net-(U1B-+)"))
 (via (at 152 60) (size 0.6) (drill 0.3) (layers "F.Cu" "B.Cu") (capping no) (covering (front no) (back no)) (plugging (front no) (back no))
  (filling no) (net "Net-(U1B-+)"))
 (via (at 148.4 48.2) (size 0.6) (drill 0.3) (layers "F.Cu" "B.Cu") (capping no) (covering (front no) (back no))
  (plugging (front no) (back no)) (filling no) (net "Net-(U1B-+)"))
 (segment (start 152.6 61.896968) (end 153.930032 63.227) (width 0.2) (layer "B.Cu") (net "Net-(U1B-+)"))
 (segment (start 153.930032 63.227) (end 156.977999 63.227) (width 0.2) (layer "B.Cu") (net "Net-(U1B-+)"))
 (segment (start 152 60.95) (end 152.6 61.55) (width 0.2) (layer "B.Cu") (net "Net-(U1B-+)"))
 (segment (start 156.977999 63.227) (end 157.68 62.524999) (width 0.2) (layer "B.Cu") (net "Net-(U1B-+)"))
 (segment (start 157.68 62.524999) (end 157.68 61.55) (width 0.2) (layer "B.Cu") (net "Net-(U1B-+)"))
 (segment (start 152 60) (end 152 60.95) (width 0.2) (layer "B.Cu") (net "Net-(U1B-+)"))
 (segment (start 146.95 48.2) (end 148.4 48.2) (width 0.2) (layer "B.Cu") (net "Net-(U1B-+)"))
 (segment (start 152.6 61.55) (end 152.6 61.896968) (width 0.2) (layer "B.Cu") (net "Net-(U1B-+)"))
 (segment (start 133.399 55.399) (end 137.6 59.6) (width 0.2) (layer "F.Cu") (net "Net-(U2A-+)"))
 (segment (start 145.599 58.399) (end 149 61.8) (width 0.2) (layer "F.Cu") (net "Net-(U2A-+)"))
 (segment (start 140.551057 58.399) (end 145.599 58.399) (width 0.2) (layer "F.Cu") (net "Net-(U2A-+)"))
 (segment (start 133.399 49.551057) (end 133.399 55.399) (width 0.2) (layer "F.Cu") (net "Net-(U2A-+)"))
 (segment (start 140.199 59.248943) (end 140.199 58.751057) (width 0.2) (layer "F.Cu") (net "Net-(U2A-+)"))
 (segment (start 145.2 48.501) (end 144.599 47.9) (width 0.2) (layer "F.Cu") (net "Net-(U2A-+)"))
 (segment (start 140.749673 59.799616) (end 140.199 59.248943) (width 0.2) (layer "F.Cu") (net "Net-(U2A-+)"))
 (segment (start 140.199 58.751057) (end 140.551057 58.399) (width 0.2) (layer "F.Cu") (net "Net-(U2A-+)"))
 (segment (start 140.775242 59.799616) (end 140.749673 59.799616) (width 0.2) (layer "F.Cu") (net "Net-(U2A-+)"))
 (segment (start 135.050057 47.9) (end 133.399 49.551057) (width 0.2) (layer "F.Cu") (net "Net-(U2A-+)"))
 (segment (start 144.599 47.9) (end 135.050057 47.9) (width 0.2) (layer "F.Cu") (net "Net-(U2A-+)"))
 (via (at 140.775242 59.799616) (size 0.6) (drill 0.3) (layers "F.Cu" "B.Cu") (capping no) (covering (front no) (back no))
  (plugging (front no) (back no)) (filling no) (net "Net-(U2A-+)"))
 (via (at 145.2 48.501) (size 0.6) (drill 0.3) (layers "F.Cu" "B.Cu") (capping no) (covering (front no) (back no))
  (plugging (front no) (back no)) (filling no) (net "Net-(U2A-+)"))
 (via (at 137.6 59.6) (size 0.6) (drill 0.3) (layers "F.Cu" "B.Cu") (capping no) (covering (front no) (back no))
  (plugging (front no) (back no)) (filling no) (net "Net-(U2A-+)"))
 (via (at 149 61.8) (size 0.6) (drill 0.3) (layers "F.Cu" "B.Cu") (capping no) (covering (front no) (back no))
  (plugging (front no) (back no)) (filling no) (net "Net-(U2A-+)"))
 (segment (start 149.81 61.8) (end 150.06 61.55) (width 0.2) (layer "B.Cu") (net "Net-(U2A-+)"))
 (segment (start 137.6 59.6) (end 138.64 59.6) (width 0.2) (layer "B.Cu") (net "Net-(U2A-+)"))
 (segment (start 144.899 48.2) (end 145.2 48.501) (width 0.2) (layer "B.Cu") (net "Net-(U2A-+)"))
 (segment (start 139.275 60.235) (end 140.339858 60.235) (width 0.2) (layer "B.Cu") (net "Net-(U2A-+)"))
 (segment (start 140.339858 60.235) (end 140.775242 59.799616) (width 0.2) (layer "B.Cu") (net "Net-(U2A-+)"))
 (segment (start 149 61.8) (end 149.81 61.8) (width 0.2) (layer "B.Cu") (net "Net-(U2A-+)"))
 (segment (start 144 48.2) (end 144.899 48.2) (width 0.2) (layer "B.Cu") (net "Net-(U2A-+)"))
 (segment (start 138.64 59.6) (end 139.275 60.235) (width 0.2) (layer "B.Cu") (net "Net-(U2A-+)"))
 (segment (start 140.8 59) (end 145 59) (width 0.2) (layer "F.Cu") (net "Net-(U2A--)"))
 (segment (start 145 59) (end 145.8 59.8) (width 0.2) (layer "F.Cu") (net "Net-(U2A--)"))
 (via (at 145.8 59.8) (size 0.6) (drill 0.3) (layers "F.Cu" "B.Cu") (capping no) (covering (front no) (back no))
  (plugging (front no) (back no)) (filling no) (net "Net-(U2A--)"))
 (via (at 140.8 59) (size 0.6) (drill 0.3) (layers "F.Cu" "B.Cu") (capping no) (covering (front no) (back no))
  (plugging (front no) (back no)) (filling no) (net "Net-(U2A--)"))
 (segment (start 140.765 58.965) (end 140.8 59) (width 0.2) (layer "B.Cu") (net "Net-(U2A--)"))
 (segment (start 139.275 58.965) (end 140.765 58.965) (width 0.2) (layer "B.Cu") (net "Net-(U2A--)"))
 (segment (start 145.8 59.8) (end 147.55 59.8) (width 0.2) (layer "B.Cu") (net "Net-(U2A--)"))
 (segment (start 140.9286 54.578543) (end 149.978543 54.578543) (width 0.2) (layer "F.Cu") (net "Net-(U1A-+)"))
 (segment (start 138.8 52.449943) (end 140.9286 54.578543) (width 0.2) (layer "F.Cu") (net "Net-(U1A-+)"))
 (segment (start 149.978543 54.578543) (end 154.6 59.2) (width 0.2) (layer "F.Cu") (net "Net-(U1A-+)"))
 (segment (start 138.8 51) (end 138.8 52.449943) (width 0.2) (layer "F.Cu") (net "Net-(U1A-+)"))
 (via (at 154.6 59.2) (size 0.6) (drill 0.3) (layers "F.Cu" "B.Cu") (capping no) (covering (front no) (back no))
  (plugging (front no) (back no)) (filling no) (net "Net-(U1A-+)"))
 (segment (start 154.6 59.2) (end 155.14 59.74) (width 0.2) (layer "B.Cu") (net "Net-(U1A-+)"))
 (segment (start 155.14 59.74) (end 155.14 61.55) (width 0.2) (layer "B.Cu") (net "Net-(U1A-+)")))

